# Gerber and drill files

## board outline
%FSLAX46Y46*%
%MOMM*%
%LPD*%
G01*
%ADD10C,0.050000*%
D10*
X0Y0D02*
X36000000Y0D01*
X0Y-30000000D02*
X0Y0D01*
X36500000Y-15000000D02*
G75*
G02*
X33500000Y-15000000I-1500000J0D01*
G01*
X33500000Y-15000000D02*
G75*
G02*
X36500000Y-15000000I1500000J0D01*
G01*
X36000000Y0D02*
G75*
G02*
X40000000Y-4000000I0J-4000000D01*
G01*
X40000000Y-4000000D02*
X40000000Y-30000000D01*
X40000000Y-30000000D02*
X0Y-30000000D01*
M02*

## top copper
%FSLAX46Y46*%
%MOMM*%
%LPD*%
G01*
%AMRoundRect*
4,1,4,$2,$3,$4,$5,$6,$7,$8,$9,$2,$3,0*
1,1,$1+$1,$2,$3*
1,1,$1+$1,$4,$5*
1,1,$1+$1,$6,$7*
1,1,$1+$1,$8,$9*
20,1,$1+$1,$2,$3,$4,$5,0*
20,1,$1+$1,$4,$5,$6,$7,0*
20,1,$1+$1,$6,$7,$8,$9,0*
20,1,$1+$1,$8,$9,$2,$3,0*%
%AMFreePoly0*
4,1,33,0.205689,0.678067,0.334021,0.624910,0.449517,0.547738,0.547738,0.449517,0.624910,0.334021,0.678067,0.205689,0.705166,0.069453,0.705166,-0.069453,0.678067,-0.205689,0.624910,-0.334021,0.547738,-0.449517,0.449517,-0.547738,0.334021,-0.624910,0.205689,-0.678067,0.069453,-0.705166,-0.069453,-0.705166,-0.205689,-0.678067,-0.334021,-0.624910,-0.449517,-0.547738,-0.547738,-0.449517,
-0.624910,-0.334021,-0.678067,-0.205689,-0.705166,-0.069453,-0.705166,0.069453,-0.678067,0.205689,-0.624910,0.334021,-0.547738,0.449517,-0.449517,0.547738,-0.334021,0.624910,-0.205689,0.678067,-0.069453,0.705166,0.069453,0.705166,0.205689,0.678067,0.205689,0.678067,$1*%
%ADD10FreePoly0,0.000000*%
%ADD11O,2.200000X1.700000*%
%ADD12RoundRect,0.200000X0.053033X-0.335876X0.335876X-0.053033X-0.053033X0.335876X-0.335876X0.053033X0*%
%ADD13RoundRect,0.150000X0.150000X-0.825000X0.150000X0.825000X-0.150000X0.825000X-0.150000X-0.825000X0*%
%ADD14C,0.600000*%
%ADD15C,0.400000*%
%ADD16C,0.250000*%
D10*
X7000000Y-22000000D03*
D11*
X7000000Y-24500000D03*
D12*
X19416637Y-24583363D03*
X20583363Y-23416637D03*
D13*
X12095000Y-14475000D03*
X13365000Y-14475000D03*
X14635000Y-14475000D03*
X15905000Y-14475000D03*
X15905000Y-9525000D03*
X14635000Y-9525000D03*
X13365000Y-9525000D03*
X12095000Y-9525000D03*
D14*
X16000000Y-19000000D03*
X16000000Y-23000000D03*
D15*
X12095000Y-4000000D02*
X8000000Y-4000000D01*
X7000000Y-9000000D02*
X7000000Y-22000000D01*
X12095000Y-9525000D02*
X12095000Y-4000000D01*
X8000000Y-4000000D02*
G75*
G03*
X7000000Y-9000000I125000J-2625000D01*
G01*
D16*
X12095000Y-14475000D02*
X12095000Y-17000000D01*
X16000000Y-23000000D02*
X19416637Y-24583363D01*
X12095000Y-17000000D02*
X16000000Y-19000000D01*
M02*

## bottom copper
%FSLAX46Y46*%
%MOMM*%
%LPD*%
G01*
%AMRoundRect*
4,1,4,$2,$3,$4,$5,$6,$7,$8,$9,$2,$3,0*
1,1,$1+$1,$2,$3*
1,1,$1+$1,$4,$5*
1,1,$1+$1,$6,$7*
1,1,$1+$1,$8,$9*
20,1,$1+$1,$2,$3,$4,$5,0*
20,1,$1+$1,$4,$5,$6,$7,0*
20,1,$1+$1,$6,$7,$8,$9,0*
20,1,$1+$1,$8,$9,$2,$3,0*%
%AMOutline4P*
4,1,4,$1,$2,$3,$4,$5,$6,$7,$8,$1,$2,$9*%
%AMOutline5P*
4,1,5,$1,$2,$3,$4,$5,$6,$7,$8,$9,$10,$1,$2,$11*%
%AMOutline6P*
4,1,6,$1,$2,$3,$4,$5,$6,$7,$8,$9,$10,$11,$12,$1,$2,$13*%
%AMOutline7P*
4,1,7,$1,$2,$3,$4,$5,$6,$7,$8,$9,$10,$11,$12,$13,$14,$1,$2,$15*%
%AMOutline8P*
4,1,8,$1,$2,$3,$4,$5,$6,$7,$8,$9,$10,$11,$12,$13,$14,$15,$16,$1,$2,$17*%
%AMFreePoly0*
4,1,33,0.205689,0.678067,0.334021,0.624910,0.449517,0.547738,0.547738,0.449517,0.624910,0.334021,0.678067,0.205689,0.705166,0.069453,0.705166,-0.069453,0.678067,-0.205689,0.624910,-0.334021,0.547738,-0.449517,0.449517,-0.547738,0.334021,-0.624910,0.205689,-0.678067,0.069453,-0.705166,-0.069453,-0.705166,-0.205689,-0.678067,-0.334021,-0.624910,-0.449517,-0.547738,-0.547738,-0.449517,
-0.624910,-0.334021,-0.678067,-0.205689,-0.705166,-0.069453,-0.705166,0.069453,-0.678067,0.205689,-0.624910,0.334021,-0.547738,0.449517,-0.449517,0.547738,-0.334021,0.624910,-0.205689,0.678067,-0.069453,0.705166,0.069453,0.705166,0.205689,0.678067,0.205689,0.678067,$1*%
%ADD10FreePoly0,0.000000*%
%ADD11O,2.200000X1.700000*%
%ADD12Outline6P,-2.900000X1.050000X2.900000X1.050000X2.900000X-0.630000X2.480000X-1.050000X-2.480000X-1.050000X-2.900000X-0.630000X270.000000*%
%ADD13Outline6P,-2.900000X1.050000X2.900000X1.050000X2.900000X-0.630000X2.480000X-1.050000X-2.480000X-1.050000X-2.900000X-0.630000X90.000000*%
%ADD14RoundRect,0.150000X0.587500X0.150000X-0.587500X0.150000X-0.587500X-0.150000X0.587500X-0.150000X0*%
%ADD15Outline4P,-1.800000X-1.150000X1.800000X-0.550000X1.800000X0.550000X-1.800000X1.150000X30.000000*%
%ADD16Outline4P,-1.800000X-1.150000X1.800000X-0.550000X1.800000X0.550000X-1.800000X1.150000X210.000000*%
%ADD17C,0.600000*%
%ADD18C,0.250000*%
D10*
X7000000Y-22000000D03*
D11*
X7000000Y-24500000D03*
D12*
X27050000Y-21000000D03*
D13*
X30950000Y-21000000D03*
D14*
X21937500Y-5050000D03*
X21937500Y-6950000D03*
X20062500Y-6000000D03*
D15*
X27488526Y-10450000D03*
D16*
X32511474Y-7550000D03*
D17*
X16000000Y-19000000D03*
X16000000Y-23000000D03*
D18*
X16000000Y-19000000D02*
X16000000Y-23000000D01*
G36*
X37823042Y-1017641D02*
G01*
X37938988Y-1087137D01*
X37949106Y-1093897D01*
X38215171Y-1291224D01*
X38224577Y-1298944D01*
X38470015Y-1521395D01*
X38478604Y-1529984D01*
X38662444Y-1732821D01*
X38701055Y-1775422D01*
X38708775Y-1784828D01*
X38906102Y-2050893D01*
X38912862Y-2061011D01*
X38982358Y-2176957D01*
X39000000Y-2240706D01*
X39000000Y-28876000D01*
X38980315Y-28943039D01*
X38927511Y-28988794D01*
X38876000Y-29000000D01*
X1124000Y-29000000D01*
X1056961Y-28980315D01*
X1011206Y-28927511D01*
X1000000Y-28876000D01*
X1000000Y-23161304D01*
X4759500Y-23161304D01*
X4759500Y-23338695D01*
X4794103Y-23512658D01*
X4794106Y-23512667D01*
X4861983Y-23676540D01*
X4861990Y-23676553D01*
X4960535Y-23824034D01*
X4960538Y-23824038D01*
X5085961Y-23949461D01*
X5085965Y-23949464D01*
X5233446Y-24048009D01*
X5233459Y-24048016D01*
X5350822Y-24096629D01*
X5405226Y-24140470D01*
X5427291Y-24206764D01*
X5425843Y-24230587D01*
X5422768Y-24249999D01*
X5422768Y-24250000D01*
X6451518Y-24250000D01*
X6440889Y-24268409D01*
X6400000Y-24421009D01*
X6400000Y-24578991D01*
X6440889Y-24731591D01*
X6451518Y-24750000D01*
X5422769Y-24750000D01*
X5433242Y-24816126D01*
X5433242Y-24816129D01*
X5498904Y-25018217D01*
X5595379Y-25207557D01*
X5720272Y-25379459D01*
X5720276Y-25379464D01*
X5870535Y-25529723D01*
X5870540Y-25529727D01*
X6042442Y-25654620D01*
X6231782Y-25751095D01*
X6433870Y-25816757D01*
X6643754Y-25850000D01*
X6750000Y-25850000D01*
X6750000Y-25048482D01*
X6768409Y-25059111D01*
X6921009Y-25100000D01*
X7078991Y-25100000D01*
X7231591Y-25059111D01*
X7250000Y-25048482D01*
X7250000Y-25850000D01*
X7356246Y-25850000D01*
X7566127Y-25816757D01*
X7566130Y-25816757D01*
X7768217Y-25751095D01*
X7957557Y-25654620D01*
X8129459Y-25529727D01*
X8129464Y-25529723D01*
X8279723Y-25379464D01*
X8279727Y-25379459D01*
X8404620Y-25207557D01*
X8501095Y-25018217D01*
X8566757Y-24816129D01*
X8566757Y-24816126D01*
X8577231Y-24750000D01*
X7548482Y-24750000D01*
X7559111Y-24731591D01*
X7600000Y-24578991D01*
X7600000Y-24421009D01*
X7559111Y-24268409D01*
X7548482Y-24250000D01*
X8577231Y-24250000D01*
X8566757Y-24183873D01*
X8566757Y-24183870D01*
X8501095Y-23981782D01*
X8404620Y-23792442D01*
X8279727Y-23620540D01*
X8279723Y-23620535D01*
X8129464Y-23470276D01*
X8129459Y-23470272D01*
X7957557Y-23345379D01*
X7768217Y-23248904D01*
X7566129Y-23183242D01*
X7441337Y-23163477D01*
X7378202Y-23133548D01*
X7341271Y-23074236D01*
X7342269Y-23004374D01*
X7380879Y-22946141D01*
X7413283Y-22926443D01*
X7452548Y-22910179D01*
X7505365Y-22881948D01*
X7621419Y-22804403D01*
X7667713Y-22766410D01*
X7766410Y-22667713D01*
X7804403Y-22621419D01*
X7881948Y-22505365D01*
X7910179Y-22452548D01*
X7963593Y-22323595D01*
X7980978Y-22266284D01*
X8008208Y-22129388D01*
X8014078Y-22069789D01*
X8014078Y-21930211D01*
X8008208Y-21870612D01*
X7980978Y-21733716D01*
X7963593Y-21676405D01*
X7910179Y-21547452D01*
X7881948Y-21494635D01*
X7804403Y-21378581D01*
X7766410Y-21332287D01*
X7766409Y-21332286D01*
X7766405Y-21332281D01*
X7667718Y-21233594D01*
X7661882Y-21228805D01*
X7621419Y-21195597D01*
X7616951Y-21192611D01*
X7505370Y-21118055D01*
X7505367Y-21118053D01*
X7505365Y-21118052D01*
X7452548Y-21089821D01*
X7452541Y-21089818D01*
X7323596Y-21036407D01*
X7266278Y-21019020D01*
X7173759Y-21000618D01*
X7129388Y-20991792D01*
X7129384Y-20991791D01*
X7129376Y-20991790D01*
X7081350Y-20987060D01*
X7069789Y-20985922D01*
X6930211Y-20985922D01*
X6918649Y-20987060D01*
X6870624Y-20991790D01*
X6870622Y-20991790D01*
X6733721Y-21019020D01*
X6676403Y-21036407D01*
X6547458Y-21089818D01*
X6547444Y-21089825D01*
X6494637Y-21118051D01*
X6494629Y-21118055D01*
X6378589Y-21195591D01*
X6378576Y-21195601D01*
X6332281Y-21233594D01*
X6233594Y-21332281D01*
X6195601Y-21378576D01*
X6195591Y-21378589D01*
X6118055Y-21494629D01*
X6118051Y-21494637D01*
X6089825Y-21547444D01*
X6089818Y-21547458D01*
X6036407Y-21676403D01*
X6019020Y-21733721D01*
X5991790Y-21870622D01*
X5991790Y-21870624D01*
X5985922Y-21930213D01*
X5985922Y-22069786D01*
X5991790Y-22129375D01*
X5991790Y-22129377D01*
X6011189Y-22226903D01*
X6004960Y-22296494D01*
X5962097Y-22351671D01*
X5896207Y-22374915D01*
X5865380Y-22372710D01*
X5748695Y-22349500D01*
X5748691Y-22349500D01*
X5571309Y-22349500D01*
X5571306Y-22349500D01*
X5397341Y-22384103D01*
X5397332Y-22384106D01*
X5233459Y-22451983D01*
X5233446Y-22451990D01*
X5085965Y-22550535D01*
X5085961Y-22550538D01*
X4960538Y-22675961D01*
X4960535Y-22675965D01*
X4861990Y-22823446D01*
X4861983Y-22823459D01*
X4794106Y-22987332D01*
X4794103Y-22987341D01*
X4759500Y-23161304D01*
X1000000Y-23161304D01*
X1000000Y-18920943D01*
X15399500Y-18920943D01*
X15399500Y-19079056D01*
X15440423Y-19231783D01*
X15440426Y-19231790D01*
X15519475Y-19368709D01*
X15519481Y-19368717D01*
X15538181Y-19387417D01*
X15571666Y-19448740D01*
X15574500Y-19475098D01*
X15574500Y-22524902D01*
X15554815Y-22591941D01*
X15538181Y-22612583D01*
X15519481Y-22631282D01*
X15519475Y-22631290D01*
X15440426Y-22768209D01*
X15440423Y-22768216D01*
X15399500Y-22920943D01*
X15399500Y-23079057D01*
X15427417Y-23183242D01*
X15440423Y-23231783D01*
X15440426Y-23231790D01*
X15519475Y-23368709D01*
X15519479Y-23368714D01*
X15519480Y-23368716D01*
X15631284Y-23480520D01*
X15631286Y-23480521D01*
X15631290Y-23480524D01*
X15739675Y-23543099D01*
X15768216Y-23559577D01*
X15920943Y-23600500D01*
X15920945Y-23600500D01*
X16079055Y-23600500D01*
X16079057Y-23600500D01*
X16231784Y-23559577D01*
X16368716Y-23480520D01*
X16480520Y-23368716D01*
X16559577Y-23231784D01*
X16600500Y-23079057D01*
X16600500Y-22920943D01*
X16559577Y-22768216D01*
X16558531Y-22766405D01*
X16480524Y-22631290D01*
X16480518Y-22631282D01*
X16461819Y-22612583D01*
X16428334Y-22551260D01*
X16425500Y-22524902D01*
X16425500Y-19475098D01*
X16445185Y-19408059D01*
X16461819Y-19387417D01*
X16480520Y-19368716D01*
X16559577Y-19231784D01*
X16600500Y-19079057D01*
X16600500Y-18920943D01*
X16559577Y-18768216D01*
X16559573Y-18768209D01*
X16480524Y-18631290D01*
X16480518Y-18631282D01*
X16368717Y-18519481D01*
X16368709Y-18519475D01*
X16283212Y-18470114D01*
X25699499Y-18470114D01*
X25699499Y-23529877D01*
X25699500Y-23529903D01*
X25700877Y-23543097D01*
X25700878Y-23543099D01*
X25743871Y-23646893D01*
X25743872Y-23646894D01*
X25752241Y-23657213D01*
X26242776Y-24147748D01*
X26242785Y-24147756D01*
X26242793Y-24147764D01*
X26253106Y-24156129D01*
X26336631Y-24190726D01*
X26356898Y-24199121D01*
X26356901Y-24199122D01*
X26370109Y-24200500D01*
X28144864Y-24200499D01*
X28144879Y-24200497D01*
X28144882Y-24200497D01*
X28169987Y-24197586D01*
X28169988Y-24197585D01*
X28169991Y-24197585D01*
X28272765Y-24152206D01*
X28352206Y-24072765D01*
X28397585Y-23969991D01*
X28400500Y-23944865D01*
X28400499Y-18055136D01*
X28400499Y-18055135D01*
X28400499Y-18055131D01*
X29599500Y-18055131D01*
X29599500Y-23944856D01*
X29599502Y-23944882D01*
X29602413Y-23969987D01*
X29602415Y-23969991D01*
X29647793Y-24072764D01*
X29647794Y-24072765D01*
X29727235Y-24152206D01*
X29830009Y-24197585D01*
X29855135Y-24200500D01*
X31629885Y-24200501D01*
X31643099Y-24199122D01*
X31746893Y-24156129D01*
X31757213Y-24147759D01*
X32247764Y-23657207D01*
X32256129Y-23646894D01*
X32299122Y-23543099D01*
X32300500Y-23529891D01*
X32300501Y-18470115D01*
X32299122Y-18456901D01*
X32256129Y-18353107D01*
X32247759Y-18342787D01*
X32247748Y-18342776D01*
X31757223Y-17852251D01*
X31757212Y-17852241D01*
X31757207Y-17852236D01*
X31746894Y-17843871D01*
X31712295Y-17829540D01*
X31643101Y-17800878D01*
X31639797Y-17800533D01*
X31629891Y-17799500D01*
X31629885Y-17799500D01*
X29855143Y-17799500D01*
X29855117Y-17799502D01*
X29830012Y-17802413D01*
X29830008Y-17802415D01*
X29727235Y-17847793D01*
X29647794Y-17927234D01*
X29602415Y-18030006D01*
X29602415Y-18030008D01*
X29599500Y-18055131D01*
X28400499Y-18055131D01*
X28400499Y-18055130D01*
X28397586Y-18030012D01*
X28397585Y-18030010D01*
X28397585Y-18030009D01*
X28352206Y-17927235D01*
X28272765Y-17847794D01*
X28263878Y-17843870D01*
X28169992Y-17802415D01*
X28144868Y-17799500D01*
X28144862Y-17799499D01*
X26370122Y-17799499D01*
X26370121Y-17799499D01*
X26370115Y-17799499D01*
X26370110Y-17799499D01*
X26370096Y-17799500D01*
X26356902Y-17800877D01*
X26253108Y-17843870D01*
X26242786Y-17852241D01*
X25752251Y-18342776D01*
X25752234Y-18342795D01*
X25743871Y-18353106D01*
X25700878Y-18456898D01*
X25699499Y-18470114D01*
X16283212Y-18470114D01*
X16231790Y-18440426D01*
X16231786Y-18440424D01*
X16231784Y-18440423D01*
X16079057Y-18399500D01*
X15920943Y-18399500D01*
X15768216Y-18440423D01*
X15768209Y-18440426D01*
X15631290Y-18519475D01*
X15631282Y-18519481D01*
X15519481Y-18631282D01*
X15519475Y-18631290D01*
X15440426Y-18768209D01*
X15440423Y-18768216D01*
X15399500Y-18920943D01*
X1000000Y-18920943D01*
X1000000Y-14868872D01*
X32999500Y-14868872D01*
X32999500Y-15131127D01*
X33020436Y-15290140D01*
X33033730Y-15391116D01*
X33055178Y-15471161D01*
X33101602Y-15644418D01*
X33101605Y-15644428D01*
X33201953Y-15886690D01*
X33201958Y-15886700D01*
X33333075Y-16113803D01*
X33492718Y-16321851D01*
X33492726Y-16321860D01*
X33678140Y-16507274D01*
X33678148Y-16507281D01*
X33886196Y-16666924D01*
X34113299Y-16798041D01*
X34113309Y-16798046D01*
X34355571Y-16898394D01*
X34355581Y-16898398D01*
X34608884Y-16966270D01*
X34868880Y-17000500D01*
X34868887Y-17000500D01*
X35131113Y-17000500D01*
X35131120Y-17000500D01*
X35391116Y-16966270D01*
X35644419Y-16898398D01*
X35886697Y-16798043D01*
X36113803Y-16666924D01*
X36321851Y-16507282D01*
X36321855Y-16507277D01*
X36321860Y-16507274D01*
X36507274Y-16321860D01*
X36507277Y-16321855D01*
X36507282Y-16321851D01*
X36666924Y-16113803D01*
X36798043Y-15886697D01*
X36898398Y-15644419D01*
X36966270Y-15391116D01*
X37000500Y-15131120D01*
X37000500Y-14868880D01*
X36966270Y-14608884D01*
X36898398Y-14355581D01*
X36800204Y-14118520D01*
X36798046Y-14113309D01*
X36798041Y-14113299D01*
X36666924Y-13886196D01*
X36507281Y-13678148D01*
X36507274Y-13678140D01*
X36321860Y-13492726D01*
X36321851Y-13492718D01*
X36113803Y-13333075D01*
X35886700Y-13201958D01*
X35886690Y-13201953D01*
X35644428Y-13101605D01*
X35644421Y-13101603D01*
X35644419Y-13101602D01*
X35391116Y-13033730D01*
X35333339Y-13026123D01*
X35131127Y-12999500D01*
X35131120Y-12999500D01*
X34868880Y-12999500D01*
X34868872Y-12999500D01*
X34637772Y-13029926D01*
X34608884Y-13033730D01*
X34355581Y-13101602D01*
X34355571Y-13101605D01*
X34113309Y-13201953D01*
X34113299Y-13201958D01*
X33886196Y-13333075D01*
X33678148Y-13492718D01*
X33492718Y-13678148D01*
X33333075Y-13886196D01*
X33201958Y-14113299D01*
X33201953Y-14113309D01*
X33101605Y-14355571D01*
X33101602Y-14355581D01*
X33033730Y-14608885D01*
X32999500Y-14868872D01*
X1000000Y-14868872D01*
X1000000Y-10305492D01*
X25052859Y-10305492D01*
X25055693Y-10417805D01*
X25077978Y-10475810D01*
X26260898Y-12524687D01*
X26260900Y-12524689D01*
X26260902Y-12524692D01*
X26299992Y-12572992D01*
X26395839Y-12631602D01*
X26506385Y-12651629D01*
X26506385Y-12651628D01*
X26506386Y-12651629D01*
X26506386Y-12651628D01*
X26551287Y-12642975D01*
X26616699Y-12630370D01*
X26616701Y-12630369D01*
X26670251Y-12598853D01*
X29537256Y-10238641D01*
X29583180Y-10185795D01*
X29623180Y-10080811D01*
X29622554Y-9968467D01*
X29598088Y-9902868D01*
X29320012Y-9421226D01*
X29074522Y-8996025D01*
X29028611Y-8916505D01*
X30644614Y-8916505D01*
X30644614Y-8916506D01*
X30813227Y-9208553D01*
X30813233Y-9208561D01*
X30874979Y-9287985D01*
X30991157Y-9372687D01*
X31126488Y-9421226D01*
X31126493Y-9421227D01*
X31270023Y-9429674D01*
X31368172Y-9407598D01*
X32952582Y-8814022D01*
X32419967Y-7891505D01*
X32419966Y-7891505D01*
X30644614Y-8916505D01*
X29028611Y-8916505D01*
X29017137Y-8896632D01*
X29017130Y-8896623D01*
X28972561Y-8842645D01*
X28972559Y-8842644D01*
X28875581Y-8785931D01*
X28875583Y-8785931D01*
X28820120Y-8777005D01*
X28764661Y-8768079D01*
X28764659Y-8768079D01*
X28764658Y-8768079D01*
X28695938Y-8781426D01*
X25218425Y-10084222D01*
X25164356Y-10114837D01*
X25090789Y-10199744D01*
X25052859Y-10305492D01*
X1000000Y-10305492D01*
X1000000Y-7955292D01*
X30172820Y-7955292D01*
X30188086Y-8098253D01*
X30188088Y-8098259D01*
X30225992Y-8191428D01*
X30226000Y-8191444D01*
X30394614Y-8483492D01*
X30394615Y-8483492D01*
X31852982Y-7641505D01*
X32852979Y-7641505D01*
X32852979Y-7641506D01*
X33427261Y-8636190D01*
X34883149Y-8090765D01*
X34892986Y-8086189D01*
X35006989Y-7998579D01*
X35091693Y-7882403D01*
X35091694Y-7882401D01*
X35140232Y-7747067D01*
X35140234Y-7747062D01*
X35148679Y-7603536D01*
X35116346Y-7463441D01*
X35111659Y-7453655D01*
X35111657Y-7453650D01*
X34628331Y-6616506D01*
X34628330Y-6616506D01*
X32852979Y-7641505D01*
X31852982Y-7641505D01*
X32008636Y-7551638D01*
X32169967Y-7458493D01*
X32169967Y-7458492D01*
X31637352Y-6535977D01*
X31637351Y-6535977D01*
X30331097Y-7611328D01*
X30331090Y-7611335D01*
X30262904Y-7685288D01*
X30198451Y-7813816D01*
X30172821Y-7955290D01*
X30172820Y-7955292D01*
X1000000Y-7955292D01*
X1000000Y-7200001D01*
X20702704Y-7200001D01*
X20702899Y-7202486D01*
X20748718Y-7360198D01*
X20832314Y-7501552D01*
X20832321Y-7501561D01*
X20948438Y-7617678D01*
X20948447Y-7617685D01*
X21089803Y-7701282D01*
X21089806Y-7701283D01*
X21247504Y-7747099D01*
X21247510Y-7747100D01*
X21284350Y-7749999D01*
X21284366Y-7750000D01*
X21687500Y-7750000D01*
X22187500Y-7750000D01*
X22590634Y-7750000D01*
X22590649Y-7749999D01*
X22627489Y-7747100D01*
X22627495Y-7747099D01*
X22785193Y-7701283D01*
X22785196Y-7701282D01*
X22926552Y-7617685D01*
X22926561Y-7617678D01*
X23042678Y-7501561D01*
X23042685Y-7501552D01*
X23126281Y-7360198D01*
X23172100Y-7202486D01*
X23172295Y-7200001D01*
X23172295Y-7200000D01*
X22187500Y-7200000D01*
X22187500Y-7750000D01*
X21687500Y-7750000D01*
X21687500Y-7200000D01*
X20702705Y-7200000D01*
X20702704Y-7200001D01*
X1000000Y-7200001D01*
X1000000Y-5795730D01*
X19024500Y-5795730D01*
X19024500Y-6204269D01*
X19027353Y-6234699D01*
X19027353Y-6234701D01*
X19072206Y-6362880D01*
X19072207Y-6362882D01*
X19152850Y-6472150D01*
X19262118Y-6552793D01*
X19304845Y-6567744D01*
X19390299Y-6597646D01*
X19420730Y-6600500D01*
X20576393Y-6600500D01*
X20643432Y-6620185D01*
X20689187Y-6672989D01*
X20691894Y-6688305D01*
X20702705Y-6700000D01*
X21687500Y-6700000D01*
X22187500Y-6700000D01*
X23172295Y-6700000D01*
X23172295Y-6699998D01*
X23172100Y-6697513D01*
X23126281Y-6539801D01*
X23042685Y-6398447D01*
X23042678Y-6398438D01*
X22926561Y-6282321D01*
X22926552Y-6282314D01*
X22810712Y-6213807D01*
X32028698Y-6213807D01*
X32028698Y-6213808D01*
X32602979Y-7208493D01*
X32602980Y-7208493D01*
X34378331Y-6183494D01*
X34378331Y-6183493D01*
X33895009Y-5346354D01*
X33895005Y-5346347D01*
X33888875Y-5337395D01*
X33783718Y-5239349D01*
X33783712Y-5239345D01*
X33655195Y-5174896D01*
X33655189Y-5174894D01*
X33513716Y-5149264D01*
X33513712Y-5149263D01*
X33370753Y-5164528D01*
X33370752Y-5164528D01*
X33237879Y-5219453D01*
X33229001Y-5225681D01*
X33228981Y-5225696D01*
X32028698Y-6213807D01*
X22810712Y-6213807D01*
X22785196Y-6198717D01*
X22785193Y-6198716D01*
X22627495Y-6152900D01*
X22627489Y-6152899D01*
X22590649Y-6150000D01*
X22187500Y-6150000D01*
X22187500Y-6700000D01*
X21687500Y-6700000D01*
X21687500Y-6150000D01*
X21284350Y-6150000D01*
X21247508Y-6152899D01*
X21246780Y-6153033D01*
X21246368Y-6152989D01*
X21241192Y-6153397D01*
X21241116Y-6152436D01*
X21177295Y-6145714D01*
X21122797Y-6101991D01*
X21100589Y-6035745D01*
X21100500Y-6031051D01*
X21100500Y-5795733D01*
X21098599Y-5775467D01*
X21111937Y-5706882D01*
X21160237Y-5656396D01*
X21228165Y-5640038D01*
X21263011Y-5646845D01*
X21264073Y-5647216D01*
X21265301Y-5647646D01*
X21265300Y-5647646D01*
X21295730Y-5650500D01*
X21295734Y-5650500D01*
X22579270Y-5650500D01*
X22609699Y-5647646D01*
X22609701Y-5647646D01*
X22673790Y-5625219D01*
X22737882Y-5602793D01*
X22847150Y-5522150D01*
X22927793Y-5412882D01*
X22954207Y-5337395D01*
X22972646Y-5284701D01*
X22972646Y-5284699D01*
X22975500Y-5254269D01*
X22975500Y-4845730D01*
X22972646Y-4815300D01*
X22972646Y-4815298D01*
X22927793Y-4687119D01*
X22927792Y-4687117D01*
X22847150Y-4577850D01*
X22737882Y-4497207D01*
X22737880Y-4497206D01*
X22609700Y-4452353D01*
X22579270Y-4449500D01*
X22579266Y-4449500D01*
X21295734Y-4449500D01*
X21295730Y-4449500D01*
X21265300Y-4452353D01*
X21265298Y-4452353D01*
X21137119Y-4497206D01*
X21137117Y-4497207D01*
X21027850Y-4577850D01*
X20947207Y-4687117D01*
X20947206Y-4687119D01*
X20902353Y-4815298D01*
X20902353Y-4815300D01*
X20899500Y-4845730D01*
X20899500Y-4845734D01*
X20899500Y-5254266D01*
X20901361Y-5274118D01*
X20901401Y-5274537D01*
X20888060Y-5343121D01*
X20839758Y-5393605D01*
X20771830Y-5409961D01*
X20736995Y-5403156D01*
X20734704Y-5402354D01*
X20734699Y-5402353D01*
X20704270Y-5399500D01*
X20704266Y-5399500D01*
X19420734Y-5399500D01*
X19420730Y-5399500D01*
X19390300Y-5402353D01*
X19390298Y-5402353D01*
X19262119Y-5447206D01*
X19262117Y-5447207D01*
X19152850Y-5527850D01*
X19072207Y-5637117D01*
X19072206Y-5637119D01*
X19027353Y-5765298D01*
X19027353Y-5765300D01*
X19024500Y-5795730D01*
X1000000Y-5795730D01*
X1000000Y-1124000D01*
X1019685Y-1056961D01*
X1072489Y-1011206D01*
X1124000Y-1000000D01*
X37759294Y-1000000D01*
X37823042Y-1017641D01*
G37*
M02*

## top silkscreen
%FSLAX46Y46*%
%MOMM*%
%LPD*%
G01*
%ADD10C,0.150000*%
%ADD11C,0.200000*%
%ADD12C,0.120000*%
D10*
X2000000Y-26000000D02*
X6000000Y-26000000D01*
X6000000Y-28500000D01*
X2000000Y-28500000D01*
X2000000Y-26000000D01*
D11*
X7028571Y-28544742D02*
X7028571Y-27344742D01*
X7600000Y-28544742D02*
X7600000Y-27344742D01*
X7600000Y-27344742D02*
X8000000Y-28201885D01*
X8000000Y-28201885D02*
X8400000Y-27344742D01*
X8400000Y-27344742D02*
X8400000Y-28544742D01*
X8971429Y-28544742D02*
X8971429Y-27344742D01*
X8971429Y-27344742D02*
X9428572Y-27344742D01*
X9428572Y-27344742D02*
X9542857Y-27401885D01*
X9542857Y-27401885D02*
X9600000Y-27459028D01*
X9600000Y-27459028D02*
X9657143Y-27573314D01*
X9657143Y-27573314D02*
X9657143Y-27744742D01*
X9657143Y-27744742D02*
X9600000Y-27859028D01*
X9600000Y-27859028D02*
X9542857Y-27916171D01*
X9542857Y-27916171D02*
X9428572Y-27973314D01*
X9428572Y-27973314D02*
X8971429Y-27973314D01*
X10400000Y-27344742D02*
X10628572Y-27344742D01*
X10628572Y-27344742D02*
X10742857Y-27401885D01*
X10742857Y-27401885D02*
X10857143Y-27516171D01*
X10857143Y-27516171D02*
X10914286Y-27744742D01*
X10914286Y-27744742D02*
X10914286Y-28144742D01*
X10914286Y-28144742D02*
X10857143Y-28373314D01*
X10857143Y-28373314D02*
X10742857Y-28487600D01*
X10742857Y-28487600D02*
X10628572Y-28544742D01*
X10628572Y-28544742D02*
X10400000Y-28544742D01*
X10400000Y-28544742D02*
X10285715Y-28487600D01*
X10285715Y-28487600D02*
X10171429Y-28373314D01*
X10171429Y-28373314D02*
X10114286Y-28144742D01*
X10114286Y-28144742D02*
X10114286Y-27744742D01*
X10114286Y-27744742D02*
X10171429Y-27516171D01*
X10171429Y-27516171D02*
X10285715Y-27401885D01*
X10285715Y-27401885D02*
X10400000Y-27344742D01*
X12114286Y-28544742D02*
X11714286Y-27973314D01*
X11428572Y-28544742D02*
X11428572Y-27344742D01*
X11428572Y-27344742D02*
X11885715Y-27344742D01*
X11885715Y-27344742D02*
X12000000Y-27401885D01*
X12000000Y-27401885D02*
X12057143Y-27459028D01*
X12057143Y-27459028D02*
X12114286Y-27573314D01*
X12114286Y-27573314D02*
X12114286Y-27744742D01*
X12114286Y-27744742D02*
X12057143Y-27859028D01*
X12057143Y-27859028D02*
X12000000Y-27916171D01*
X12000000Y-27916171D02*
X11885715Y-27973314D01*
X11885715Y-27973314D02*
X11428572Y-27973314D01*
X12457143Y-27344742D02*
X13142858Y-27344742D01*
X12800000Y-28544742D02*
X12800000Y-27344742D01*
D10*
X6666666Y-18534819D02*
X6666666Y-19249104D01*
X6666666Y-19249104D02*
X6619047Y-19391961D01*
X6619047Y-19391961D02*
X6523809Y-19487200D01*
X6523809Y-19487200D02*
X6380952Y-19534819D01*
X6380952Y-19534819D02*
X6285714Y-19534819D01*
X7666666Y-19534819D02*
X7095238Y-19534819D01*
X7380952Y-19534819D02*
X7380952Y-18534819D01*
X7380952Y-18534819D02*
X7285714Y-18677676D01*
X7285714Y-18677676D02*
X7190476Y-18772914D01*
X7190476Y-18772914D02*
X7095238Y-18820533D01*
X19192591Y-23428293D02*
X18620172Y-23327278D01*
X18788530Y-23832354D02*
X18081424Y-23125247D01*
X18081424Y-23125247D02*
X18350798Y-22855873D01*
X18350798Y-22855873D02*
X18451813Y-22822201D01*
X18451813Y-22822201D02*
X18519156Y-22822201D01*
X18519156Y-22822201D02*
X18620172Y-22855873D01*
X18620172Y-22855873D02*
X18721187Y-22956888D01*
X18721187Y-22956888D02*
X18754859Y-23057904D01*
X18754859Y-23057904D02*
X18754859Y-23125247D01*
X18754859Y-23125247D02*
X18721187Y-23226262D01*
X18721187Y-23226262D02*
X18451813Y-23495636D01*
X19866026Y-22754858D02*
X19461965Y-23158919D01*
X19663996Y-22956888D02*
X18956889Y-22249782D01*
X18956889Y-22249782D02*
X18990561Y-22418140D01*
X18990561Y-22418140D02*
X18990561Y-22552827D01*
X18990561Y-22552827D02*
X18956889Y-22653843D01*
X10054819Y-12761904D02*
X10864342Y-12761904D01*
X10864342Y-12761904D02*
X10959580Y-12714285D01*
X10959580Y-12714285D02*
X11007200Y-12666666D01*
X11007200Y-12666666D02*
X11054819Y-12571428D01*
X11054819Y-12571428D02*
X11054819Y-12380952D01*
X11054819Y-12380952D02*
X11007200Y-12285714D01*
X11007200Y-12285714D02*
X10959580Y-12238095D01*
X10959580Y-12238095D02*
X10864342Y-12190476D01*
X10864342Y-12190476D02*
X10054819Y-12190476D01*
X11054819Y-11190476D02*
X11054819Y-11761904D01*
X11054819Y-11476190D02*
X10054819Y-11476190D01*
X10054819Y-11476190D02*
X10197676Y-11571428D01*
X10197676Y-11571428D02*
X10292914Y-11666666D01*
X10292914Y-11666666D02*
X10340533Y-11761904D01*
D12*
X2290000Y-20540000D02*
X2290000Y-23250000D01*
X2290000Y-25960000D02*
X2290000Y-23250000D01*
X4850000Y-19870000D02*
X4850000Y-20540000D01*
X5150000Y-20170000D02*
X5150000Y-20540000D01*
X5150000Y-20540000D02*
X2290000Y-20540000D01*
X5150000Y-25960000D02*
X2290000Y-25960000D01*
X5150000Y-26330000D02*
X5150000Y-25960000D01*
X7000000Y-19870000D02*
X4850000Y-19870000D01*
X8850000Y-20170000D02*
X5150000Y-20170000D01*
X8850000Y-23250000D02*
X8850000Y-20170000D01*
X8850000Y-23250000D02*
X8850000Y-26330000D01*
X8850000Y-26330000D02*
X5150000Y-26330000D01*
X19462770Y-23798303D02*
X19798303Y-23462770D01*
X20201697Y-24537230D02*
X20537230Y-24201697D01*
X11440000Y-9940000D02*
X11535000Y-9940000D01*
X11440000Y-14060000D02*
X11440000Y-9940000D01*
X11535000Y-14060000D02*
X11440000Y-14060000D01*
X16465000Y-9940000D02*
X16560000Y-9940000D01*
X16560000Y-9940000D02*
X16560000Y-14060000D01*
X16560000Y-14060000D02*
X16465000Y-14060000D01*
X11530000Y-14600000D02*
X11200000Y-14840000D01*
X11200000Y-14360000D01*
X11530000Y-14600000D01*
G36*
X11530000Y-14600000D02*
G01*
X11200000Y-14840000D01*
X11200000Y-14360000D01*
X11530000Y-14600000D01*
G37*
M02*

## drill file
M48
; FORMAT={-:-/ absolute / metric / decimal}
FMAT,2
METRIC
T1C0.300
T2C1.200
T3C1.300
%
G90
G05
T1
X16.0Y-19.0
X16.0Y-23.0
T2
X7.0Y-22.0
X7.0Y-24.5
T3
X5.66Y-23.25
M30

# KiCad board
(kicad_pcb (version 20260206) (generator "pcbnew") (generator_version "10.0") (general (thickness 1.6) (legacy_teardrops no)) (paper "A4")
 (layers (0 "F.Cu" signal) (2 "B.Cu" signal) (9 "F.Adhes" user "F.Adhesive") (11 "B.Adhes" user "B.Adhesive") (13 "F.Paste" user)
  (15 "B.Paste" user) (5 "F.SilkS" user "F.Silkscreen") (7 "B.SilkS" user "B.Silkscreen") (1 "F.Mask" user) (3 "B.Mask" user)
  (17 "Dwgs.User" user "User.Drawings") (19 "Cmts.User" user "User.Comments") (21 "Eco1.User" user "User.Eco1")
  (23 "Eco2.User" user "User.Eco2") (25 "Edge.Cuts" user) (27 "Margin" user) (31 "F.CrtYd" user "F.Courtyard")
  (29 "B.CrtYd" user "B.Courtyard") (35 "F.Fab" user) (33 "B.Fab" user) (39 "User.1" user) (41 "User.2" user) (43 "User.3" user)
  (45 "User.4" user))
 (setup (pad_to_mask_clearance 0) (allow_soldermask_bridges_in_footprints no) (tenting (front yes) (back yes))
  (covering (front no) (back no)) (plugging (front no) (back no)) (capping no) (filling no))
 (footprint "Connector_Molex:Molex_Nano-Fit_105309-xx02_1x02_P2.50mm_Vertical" (layer "F.Cu") (at 7 22)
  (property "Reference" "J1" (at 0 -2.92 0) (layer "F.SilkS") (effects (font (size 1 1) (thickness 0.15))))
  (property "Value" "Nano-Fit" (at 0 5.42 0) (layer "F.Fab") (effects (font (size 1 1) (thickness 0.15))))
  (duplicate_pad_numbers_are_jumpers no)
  (fp_line (start -4.71 -1.46) (end -4.71 1.25) (stroke (width 0.12) (type solid)) (layer "F.SilkS"))
  (fp_line (start -4.71 3.96) (end -4.71 1.25) (stroke (width 0.12) (type solid)) (layer "F.SilkS"))
  (fp_line (start -2.15 -2.13) (end -2.15 -1.46) (stroke (width 0.12) (type solid)) (layer "F.SilkS"))
  (fp_line (start -1.85 -1.83) (end -1.85 -1.46) (stroke (width 0.12) (type solid)) (layer "F.SilkS"))
  (fp_line (start -1.85 -1.46) (end -4.71 -1.46) (stroke (width 0.12) (type solid)) (layer "F.SilkS"))
  (fp_line (start -1.85 3.96) (end -4.71 3.96) (stroke (width 0.12) (type solid)) (layer "F.SilkS"))
  (fp_line (start -1.85 4.33) (end -1.85 3.96) (stroke (width 0.12) (type solid)) (layer "F.SilkS"))
  (fp_line (start 0 -2.13) (end -2.15 -2.13) (stroke (width 0.12) (type solid)) (layer "F.SilkS"))
  (fp_line (start 1.85 -1.83) (end -1.85 -1.83) (stroke (width 0.12) (type solid)) (layer "F.SilkS"))
  (fp_line (start 1.85 1.25) (end 1.85 -1.83) (stroke (width 0.12) (type solid)) (layer "F.SilkS"))
  (fp_line (start 1.85 1.25) (end 1.85 4.33) (stroke (width 0.12) (type solid)) (layer "F.SilkS"))
  (fp_line (start 1.85 4.33) (end -1.85 4.33) (stroke (width 0.12) (type solid)) (layer "F.SilkS"))
  (pad "" np_thru_hole circle (at -1.34 1.25) (size 1.3 1.3) (drill 1.3) (layers "*.Cu" "*.Mask"))
  (pad "1" thru_hole custom (at 0 0) (size 1.417157 1.417157) (drill 1.2) (layers "*.Cu" "*.Mask") (remove_unused_layers no) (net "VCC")
   (options (clearance outline) (anchor circle)) (primitives))
  (pad "2" thru_hole oval (at 0 2.5) (size 2.2 1.7) (drill 1.2) (layers "*.Cu" "*.Mask") (remove_unused_layers no) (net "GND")))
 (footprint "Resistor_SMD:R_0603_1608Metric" (layer "F.Cu") (at 20 24 45)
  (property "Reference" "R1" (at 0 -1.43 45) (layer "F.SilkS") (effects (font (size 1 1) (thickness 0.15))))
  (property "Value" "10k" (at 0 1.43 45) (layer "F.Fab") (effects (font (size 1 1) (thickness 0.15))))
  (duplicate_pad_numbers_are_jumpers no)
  (fp_line (start -0.237258 -0.5225) (end 0.237258 -0.5225) (stroke (width 0.12) (type solid)) (layer "F.SilkS"))
  (fp_line (start -0.237258 0.5225) (end 0.237258 0.5225) (stroke (width 0.12) (type solid)) (layer "F.SilkS"))
  (pad "1" smd roundrect (at -0.825 0 45) (size 0.8 0.95) (layers "F.Cu" "F.Mask" "F.Paste") (roundrect_rratio 0.25) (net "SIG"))
  (pad "2" smd roundrect (at 0.825 0 45) (size 0.8 0.95) (layers "F.Cu" "F.Mask" "F.Paste") (roundrect_rratio 0.25) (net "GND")))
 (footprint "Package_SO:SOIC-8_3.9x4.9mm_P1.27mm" (layer "F.Cu") (at 14 12 90)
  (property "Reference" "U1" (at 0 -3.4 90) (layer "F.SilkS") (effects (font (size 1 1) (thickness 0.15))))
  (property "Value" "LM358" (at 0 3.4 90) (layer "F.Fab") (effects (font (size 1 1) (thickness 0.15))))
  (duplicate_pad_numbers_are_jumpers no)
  (fp_line (start 2.06 -2.56) (end 2.06 -2.465) (stroke (width 0.12) (type solid)) (layer "F.SilkS"))
  (fp_line (start -2.06 -2.56) (end 2.06 -2.56) (stroke (width 0.12) (type solid)) (layer "F.SilkS"))
  (fp_line (start -2.06 -2.465) (end -2.06 -2.56) (stroke (width 0.12) (type solid)) (layer "F.SilkS"))
  (fp_line (start 2.06 2.465) (end 2.06 2.56) (stroke (width 0.12) (type solid)) (layer "F.SilkS"))
  (fp_line (start 2.06 2.56) (end -2.06 2.56) (stroke (width 0.12) (type solid)) (layer "F.SilkS"))
  (fp_line (start -2.06 2.56) (end -2.06 2.465) (stroke (width 0.12) (type solid)) (layer "F.SilkS"))
  (fp_poly (pts (xy -2.6 -2.47) (xy -2.84 -2.8) (xy -2.36 -2.8)) (stroke (width 0.12) (type solid)) (fill yes) (layer "F.SilkS"))
  (pad "1" smd roundrect (at -2.475 -1.905 90) (size 1.95 0.6) (layers "F.Cu" "F.Mask" "F.Paste") (roundrect_rratio 0.25) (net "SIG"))
  (pad "2" smd roundrect (at -2.475 -0.635 90) (size 1.95 0.6) (layers "F.Cu" "F.Mask" "F.Paste") (roundrect_rratio 0.25))
  (pad "3" smd roundrect (at -2.475 0.635 90) (size 1.95 0.6) (layers "F.Cu" "F.Mask" "F.Paste") (roundrect_rratio 0.25))
  (pad "4" smd roundrect (at -2.475 1.905 90) (size 1.95 0.6) (layers "F.Cu" "F.Mask" "F.Paste") (roundrect_rratio 0.25) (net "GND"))
  (pad "5" smd roundrect (at 2.475 1.905 90) (size 1.95 0.6) (layers "F.Cu" "F.Mask" "F.Paste") (roundrect_rratio 0.25))
  (pad "6" smd roundrect (at 2.475 0.635 90) (size 1.95 0.6) (layers "F.Cu" "F.Mask" "F.Paste") (roundrect_rratio 0.25))
  (pad "7" smd roundrect (at 2.475 -0.635 90) (size 1.95 0.6) (layers "F.Cu" "F.Mask" "F.Paste") (roundrect_rratio 0.25))
  (pad "8" smd roundrect (at 2.475 -1.905 90) (size 1.95 0.6) (layers "F.Cu" "F.Mask" "F.Paste") (roundrect_rratio 0.25) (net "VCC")))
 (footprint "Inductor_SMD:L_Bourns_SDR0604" (layer "B.Cu") (at 29 21 -90)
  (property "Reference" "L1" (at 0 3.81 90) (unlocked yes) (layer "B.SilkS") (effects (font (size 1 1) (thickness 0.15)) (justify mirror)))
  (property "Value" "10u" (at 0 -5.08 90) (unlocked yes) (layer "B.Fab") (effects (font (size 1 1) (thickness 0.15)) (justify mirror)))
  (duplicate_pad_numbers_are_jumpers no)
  (pad "1" smd roundrect (at 0 1.95 270) (size 5.8 2.1) (layers "B.Cu" "B.Mask" "B.Paste") (roundrect_rratio 0) (chamfer_ratio 0.2)
   (chamfer bottom_left bottom_right) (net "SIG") (die_length 2))
  (pad "2" smd roundrect (at 0 -1.95 90) (size 5.8 2.1) (layers "B.Cu" "B.Mask" "B.Paste") (roundrect_rratio 0) (chamfer_ratio 0.2)
   (chamfer bottom_left bottom_right) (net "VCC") (die_length 2)))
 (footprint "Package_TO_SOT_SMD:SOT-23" (layer "B.Cu") (at 21 6 180)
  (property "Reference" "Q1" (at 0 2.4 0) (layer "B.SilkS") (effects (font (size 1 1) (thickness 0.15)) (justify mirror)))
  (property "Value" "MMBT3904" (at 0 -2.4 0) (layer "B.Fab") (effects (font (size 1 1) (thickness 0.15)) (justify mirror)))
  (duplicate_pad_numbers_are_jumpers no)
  (pad "1" smd roundrect (at -0.9375 0.95 180) (size 1.475 0.6) (layers "B.Cu" "B.Mask" "B.Paste") (roundrect_rratio 0.25) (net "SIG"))
  (pad "2" smd roundrect (at -0.9375 -0.95 180) (size 1.475 0.6) (layers "B.Cu" "B.Mask" "B.Paste") (roundrect_rratio 0.25) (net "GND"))
  (pad "3" smd roundrect (at 0.9375 0 180) (size 1.475 0.6) (layers "B.Cu" "B.Mask" "B.Paste") (roundrect_rratio 0.25)))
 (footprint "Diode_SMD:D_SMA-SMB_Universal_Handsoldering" (layer "B.Cu") (at 30 9 30)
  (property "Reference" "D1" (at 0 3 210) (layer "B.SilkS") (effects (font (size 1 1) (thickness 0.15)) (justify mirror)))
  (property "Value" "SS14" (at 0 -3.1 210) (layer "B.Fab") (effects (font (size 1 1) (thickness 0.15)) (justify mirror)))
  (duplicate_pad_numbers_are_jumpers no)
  (pad "1" smd trapezoid (at -2.9 0 30) (size 3.6 1.7) (rect_delta 0.6 0) (layers "B.Cu" "B.Mask" "B.Paste") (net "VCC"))
  (pad "2" smd trapezoid (at 2.9 0 210) (size 3.6 1.7) (rect_delta 0.6 0) (layers "B.Cu" "B.Mask" "B.Paste") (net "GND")))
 (gr_rect (start 2 26) (end 6 28.5) (stroke (width 0.15) (type default)) (fill no) (layer "F.SilkS"))
 (gr_line (start 0 0) (end 36 0) (stroke (width 0.05) (type default)) (layer "Edge.Cuts"))
 (gr_line (start 0 30) (end 0 0) (stroke (width 0.05) (type default)) (layer "Edge.Cuts"))
 (gr_circle (center 35 15) (end 36.5 15) (stroke (width 0.05) (type default)) (fill no) (layer "Edge.Cuts"))
 (gr_arc (start 36 0) (mid 38.828427 1.171572) (end 40 4) (stroke (width 0.05) (type default)) (layer "Edge.Cuts"))
 (gr_line (start 40 4) (end 40 30) (stroke (width 0.05) (type default)) (layer "Edge.Cuts"))
 (gr_line (start 40 30) (end 0 30) (stroke (width 0.05) (type default)) (layer "Edge.Cuts"))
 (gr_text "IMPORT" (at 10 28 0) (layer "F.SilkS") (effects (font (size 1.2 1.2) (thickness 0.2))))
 (segment (start 12.095 4) (end 8 4) (width 0.4) (layer "F.Cu") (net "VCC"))
 (segment (start 7 9) (end 7 22) (width 0.4) (layer "F.Cu") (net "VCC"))
 (segment (start 12.095 9.525) (end 12.095 4) (width 0.4) (layer "F.Cu") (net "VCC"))
 (arc (start 8 4) (mid 5.5 6.5) (end 7 9) (width 0.4) (layer "F.Cu") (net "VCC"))
 (segment (start 12.095 14.475) (end 12.095 17) (width 0.25) (layer "F.Cu") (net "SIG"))
 (segment (start 16 23) (end 19.416637 24.583363) (width 0.25) (layer "F.Cu") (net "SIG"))
 (segment (start 12.095 17) (end 16 19) (width 0.25) (layer "F.Cu") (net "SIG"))
 (via (at 16 19) (size 0.6) (drill 0.3) (layers "F.Cu" "B.Cu") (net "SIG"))
 (via (at 16 23) (size 0.6) (drill 0.3) (layers "F.Cu" "B.Cu") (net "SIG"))
 (segment (start 16 19) (end 16 23) (width 0.25) (layer "B.Cu") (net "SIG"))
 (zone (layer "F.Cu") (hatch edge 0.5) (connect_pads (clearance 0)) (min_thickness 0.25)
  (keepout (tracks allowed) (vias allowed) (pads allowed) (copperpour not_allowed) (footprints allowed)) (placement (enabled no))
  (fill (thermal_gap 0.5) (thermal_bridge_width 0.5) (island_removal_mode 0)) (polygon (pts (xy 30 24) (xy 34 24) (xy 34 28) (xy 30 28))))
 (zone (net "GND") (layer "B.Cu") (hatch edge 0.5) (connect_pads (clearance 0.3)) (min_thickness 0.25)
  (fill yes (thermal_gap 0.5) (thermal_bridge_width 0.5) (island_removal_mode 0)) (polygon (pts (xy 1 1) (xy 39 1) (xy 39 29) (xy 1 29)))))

